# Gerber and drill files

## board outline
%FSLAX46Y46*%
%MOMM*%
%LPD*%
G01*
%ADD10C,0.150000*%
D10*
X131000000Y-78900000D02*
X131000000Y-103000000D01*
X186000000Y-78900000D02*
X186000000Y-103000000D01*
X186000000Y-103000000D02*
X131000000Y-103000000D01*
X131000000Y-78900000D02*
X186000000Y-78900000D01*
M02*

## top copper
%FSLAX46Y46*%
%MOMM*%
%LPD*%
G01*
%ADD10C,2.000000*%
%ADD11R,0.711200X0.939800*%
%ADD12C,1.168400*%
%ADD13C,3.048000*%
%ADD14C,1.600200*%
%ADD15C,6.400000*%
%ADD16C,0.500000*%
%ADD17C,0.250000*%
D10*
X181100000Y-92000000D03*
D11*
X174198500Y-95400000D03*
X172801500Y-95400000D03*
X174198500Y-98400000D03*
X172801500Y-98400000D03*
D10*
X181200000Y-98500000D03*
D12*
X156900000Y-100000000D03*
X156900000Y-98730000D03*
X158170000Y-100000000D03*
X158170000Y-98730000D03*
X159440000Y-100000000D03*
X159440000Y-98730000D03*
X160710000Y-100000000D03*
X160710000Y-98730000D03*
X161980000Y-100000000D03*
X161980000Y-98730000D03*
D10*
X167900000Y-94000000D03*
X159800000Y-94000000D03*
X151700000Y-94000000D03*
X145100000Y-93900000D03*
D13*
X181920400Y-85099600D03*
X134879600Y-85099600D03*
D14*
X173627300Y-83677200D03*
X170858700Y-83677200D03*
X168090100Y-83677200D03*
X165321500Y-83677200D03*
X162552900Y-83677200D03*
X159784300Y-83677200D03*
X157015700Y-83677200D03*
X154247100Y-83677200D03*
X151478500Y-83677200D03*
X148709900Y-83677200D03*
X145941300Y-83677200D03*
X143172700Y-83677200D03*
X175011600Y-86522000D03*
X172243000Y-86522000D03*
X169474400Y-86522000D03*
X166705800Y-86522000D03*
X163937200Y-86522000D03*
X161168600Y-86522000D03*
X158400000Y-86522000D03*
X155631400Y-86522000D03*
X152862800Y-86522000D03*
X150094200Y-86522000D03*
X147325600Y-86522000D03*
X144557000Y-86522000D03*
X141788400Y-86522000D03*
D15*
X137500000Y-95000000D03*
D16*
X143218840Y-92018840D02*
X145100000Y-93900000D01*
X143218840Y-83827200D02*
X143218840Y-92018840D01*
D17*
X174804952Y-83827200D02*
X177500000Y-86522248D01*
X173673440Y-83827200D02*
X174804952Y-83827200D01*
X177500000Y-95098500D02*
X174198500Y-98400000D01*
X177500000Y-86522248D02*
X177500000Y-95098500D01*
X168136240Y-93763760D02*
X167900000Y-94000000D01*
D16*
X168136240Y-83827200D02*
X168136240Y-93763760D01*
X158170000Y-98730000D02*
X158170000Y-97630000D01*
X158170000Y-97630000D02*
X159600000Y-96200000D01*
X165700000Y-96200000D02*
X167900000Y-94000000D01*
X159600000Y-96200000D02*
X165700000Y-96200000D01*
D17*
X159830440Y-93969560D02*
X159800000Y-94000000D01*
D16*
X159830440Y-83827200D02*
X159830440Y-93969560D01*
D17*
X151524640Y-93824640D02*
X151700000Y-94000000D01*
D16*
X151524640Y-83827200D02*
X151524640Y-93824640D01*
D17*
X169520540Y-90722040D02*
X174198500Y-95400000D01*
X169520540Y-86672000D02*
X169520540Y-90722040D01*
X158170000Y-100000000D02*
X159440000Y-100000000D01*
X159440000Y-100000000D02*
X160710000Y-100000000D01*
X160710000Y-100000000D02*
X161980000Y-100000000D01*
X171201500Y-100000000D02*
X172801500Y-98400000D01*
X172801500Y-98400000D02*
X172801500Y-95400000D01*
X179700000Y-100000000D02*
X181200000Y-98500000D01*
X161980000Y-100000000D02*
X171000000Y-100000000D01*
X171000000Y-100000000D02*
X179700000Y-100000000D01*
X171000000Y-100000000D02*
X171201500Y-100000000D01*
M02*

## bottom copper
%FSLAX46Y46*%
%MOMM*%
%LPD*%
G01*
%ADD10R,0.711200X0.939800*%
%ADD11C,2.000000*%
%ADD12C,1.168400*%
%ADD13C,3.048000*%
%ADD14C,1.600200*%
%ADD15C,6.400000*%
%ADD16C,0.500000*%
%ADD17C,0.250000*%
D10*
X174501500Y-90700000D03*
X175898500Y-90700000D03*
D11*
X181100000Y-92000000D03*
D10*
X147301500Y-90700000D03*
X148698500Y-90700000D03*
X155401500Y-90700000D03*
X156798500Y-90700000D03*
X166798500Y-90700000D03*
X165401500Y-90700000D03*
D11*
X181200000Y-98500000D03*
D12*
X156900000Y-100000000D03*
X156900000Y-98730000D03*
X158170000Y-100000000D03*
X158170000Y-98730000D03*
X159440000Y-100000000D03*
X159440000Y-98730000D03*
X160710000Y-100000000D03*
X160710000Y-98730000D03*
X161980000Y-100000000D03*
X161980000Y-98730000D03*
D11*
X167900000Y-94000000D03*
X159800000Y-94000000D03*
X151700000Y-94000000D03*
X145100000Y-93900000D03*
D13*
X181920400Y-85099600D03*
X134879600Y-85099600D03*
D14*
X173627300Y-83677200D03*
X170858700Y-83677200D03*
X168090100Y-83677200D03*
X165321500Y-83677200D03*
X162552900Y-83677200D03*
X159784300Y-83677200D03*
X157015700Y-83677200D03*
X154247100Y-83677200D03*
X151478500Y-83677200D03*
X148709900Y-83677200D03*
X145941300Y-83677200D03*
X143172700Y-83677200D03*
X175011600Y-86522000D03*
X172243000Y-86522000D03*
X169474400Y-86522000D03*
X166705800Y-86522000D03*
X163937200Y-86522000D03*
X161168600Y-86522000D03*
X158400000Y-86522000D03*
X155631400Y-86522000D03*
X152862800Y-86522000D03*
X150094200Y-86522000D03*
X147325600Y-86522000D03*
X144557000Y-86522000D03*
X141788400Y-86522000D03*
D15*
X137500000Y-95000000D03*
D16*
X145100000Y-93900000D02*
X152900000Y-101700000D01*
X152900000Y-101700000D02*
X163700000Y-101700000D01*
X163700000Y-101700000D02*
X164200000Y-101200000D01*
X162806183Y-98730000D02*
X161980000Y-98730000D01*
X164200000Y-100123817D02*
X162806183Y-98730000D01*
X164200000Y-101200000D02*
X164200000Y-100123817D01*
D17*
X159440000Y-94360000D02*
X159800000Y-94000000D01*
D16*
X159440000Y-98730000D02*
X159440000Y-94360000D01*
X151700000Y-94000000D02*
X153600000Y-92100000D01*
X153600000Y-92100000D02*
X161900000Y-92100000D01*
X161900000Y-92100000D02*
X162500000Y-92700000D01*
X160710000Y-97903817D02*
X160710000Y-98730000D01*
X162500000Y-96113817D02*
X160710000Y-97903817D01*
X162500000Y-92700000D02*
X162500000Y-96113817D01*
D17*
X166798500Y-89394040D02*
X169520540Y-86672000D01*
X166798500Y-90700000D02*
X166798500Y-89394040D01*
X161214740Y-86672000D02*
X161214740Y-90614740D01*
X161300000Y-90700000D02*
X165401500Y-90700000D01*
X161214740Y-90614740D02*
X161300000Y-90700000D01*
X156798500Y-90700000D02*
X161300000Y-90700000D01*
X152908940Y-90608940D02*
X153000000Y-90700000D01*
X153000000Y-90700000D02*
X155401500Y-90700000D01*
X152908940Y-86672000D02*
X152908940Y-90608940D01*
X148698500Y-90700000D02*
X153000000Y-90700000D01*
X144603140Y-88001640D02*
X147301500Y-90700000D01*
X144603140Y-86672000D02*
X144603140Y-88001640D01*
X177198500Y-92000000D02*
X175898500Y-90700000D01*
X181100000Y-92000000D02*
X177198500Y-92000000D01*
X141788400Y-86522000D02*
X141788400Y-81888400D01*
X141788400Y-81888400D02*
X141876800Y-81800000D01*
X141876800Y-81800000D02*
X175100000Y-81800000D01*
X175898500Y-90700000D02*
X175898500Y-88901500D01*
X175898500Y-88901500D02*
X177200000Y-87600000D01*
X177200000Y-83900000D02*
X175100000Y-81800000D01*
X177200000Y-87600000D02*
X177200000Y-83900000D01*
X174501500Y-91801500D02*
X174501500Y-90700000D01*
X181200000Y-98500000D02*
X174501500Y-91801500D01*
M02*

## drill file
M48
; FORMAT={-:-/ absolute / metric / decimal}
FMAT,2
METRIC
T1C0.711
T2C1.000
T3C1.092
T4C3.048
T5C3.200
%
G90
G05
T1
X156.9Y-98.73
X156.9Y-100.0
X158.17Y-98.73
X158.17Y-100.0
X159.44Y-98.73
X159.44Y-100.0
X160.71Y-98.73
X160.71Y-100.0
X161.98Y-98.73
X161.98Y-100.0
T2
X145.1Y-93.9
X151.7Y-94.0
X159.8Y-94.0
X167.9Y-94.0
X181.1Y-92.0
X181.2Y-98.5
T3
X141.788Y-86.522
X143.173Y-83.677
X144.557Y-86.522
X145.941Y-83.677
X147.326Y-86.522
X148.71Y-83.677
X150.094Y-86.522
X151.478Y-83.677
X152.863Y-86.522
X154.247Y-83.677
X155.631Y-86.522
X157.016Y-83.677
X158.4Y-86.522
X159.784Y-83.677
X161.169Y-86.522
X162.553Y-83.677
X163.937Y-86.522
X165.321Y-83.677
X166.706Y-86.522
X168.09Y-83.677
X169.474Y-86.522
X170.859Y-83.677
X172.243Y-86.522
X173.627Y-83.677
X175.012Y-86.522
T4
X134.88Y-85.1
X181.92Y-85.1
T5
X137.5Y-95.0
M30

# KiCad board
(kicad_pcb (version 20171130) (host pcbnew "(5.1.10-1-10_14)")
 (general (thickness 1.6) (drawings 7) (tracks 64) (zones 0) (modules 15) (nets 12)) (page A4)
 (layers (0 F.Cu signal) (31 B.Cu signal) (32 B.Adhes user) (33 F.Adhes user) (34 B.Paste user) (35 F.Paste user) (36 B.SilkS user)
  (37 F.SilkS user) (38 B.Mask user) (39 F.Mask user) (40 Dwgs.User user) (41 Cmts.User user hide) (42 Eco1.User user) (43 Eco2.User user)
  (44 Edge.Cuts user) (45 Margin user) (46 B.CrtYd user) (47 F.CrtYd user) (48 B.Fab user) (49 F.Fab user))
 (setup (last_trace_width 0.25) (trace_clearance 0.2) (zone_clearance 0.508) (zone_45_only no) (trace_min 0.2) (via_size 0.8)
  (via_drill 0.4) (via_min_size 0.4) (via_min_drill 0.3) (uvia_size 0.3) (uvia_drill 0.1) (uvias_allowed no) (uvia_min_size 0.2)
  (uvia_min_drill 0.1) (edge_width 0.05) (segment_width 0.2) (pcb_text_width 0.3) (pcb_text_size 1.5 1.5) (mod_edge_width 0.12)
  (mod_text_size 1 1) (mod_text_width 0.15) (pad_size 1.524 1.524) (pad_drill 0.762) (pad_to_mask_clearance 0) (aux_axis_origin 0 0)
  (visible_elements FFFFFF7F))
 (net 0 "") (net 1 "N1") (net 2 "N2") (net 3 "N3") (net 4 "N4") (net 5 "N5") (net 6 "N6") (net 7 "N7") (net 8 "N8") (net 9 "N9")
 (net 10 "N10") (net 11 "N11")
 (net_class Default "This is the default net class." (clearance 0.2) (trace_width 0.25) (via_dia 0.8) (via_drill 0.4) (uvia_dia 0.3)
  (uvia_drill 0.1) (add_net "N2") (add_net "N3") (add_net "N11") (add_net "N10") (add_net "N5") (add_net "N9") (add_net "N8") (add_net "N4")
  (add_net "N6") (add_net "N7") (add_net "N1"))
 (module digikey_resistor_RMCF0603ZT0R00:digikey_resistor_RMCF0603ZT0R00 (layer B.Cu) (at 175.2 90.7 180)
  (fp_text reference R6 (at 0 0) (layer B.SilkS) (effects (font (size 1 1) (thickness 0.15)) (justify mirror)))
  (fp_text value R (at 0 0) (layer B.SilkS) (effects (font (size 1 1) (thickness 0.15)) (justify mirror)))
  (pad 2 smd rect (at 0.6985 0 180) (size 0.7112 0.9398) (layers B.Cu B.Paste B.Mask) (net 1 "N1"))
  (pad 1 smd rect (at -0.6985 0 180) (size 0.7112 0.9398) (layers B.Cu B.Paste B.Mask) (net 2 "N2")))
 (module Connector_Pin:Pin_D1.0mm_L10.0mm (layer F.Cu) (at 181.1 92)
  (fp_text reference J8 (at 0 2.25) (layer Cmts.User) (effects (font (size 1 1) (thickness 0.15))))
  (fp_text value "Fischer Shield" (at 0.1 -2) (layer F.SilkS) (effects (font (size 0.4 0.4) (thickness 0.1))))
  (pad 1 thru_hole circle (at 0 0) (size 2 2) (drill 1) (layers *.Cu *.Mask) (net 2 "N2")))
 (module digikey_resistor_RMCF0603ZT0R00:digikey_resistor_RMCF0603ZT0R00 (layer F.Cu) (at 173.5 95.4)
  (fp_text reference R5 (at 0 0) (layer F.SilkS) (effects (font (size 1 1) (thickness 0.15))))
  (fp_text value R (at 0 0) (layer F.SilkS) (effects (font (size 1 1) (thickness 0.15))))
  (pad 2 smd rect (at 0.6985 0) (size 0.7112 0.9398) (layers F.Cu F.Paste F.Mask) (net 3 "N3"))
  (pad 1 smd rect (at -0.6985 0) (size 0.7112 0.9398) (layers F.Cu F.Paste F.Mask) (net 1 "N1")))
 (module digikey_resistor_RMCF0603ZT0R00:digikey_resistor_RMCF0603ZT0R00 (layer F.Cu) (at 173.5 98.4)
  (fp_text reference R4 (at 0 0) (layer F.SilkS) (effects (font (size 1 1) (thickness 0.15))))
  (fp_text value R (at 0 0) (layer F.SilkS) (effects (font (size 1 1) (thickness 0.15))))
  (pad 2 smd rect (at 0.6985 0) (size 0.7112 0.9398) (layers F.Cu F.Paste F.Mask) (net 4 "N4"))
  (pad 1 smd rect (at -0.6985 0) (size 0.7112 0.9398) (layers F.Cu F.Paste F.Mask) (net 1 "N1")))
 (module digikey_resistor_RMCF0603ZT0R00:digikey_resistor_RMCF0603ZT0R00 (layer B.Cu) (at 148 90.7 180)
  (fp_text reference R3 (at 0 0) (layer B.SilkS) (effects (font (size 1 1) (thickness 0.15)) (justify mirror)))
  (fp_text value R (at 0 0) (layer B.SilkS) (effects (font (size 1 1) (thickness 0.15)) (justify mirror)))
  (pad 2 smd rect (at 0.6985 0 180) (size 0.7112 0.9398) (layers B.Cu B.Paste B.Mask) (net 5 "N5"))
  (pad 1 smd rect (at -0.6985 0 180) (size 0.7112 0.9398) (layers B.Cu B.Paste B.Mask) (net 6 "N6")))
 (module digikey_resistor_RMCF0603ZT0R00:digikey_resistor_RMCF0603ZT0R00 (layer B.Cu) (at 156.1 90.7 180)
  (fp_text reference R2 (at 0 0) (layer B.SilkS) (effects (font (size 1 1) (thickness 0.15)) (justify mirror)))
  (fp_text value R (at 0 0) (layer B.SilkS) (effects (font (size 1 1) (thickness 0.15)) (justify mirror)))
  (pad 2 smd rect (at 0.6985 0 180) (size 0.7112 0.9398) (layers B.Cu B.Paste B.Mask) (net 6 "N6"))
  (pad 1 smd rect (at -0.6985 0 180) (size 0.7112 0.9398) (layers B.Cu B.Paste B.Mask) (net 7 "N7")))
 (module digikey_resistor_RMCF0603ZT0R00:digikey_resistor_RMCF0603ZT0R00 (layer B.Cu) (at 166.1 90.7)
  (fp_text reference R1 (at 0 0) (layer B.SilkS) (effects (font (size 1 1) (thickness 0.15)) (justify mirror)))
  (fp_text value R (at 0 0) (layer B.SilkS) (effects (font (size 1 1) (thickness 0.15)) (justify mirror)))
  (pad 2 smd rect (at 0.6985 0) (size 0.7112 0.9398) (layers B.Cu B.Paste B.Mask) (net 3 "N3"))
  (pad 1 smd rect (at -0.6985 0) (size 0.7112 0.9398) (layers B.Cu B.Paste B.Mask) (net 7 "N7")))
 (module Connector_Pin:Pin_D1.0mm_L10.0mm (layer F.Cu) (at 181.2 98.5)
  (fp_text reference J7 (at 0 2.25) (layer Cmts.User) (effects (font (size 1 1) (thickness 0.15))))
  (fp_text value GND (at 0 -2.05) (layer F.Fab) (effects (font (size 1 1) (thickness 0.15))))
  (pad 1 thru_hole circle (at 0 0) (size 2 2) (drill 1) (layers *.Cu *.Mask) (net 1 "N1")))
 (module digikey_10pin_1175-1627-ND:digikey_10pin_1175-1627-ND (layer F.Cu) (at 156.9 100)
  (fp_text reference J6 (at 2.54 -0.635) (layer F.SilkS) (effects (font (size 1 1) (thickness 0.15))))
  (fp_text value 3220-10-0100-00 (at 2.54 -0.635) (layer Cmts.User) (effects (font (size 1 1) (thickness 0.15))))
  (pad 1 thru_hole circle (at 0 0) (size 1.1684 1.1684) (drill 0.7112) (layers *.Cu *.Mask))
  (pad 2 thru_hole circle (at 0 -1.27) (size 1.1684 1.1684) (drill 0.7112) (layers *.Cu *.Mask))
  (pad 3 thru_hole circle (at 1.27 0) (size 1.1684 1.1684) (drill 0.7112) (layers *.Cu *.Mask) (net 1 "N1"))
  (pad 4 thru_hole circle (at 1.27 -1.27) (size 1.1684 1.1684) (drill 0.7112) (layers *.Cu *.Mask) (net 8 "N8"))
  (pad 5 thru_hole circle (at 2.54 0) (size 1.1684 1.1684) (drill 0.7112) (layers *.Cu *.Mask) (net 1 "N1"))
  (pad 6 thru_hole circle (at 2.54 -1.27) (size 1.1684 1.1684) (drill 0.7112) (layers *.Cu *.Mask) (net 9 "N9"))
  (pad 7 thru_hole circle (at 3.81 0) (size 1.1684 1.1684) (drill 0.7112) (layers *.Cu *.Mask) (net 1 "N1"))
  (pad 8 thru_hole circle (at 3.81 -1.27) (size 1.1684 1.1684) (drill 0.7112) (layers *.Cu *.Mask) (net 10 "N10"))
  (pad 9 thru_hole circle (at 5.08 0) (size 1.1684 1.1684) (drill 0.7112) (layers *.Cu *.Mask) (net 1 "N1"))
  (pad 10 thru_hole circle (at 5.08 -1.27) (size 1.1684 1.1684) (drill 0.7112) (layers *.Cu *.Mask) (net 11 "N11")))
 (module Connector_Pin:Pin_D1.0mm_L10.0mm (layer F.Cu) (at 167.9 94)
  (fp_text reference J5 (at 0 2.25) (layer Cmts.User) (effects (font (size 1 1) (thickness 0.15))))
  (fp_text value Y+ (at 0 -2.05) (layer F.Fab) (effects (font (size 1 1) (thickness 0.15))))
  (pad 1 thru_hole circle (at 0 0) (size 2 2) (drill 1) (layers *.Cu *.Mask) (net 8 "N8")))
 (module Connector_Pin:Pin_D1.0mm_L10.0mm (layer F.Cu) (at 159.8 94)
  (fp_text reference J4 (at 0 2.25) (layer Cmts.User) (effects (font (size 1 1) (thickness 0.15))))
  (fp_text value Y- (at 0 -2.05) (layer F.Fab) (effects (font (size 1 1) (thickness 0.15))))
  (pad 1 thru_hole circle (at 0 0) (size 2 2) (drill 1) (layers *.Cu *.Mask) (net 9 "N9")))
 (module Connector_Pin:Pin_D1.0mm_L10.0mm (layer F.Cu) (at 151.7 94)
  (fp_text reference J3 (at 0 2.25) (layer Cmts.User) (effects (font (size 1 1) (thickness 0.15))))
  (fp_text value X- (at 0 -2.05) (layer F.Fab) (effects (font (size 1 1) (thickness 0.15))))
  (pad 1 thru_hole circle (at 0 0) (size 2 2) (drill 1) (layers *.Cu *.Mask) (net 10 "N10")))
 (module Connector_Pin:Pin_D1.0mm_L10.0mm (layer F.Cu) (at 145.1 93.9)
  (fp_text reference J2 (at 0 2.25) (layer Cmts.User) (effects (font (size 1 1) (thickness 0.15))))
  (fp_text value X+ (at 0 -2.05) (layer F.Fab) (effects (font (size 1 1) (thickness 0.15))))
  (pad 1 thru_hole circle (at 0 0) (size 2 2) (drill 1) (layers *.Cu *.Mask) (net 11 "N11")))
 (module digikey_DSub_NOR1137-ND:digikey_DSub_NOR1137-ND (layer F.Cu) (at 158.4 75.6)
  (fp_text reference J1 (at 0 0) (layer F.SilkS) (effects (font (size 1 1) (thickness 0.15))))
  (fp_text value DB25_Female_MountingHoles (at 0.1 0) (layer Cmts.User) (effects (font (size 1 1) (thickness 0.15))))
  (pad 27 thru_hole circle (at 23.5204 9.4996) (size 3.048 3.048) (drill 3.048) (layers *.Cu *.Mask))
  (pad 26 thru_hole circle (at -23.5204 9.4996) (size 3.048 3.048) (drill 3.048) (layers *.Cu *.Mask))
  (pad 25 thru_hole circle (at 15.2273 8.0772) (size 1.6002 1.6002) (drill 1.0922) (layers *.Cu *.Mask) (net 4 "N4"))
  (pad 24 thru_hole circle (at 12.4587 8.0772) (size 1.6002 1.6002) (drill 1.0922) (layers *.Cu *.Mask))
  (pad 23 thru_hole circle (at 9.6901 8.0772) (size 1.6002 1.6002) (drill 1.0922) (layers *.Cu *.Mask) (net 8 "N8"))
  (pad 22 thru_hole circle (at 6.9215 8.0772) (size 1.6002 1.6002) (drill 1.0922) (layers *.Cu *.Mask))
  (pad 21 thru_hole circle (at 4.1529 8.0772) (size 1.6002 1.6002) (drill 1.0922) (layers *.Cu *.Mask))
  (pad 20 thru_hole circle (at 1.3843 8.0772) (size 1.6002 1.6002) (drill 1.0922) (layers *.Cu *.Mask) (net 9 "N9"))
  (pad 19 thru_hole circle (at -1.3843 8.0772) (size 1.6002 1.6002) (drill 1.0922) (layers *.Cu *.Mask))
  (pad 18 thru_hole circle (at -4.1529 8.0772) (size 1.6002 1.6002) (drill 1.0922) (layers *.Cu *.Mask))
  (pad 17 thru_hole circle (at -6.9215 8.0772) (size 1.6002 1.6002) (drill 1.0922) (layers *.Cu *.Mask) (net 10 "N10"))
  (pad 16 thru_hole circle (at -9.6901 8.0772) (size 1.6002 1.6002) (drill 1.0922) (layers *.Cu *.Mask))
  (pad 15 thru_hole circle (at -12.4587 8.0772) (size 1.6002 1.6002) (drill 1.0922) (layers *.Cu *.Mask))
  (pad 14 thru_hole circle (at -15.2273 8.0772) (size 1.6002 1.6002) (drill 1.0922) (layers *.Cu *.Mask) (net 11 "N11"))
  (pad 13 thru_hole circle (at 16.6116 10.922) (size 1.6002 1.6002) (drill 1.0922) (layers *.Cu *.Mask))
  (pad 12 thru_hole circle (at 13.843 10.922) (size 1.6002 1.6002) (drill 1.0922) (layers *.Cu *.Mask))
  (pad 11 thru_hole circle (at 11.0744 10.922) (size 1.6002 1.6002) (drill 1.0922) (layers *.Cu *.Mask) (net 3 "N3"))
  (pad 10 thru_hole circle (at 8.3058 10.922) (size 1.6002 1.6002) (drill 1.0922) (layers *.Cu *.Mask))
  (pad 9 thru_hole circle (at 5.5372 10.922) (size 1.6002 1.6002) (drill 1.0922) (layers *.Cu *.Mask))
  (pad 8 thru_hole circle (at 2.7686 10.922) (size 1.6002 1.6002) (drill 1.0922) (layers *.Cu *.Mask) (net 7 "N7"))
  (pad 7 thru_hole circle (at 0 10.922) (size 1.6002 1.6002) (drill 1.0922) (layers *.Cu *.Mask))
  (pad 6 thru_hole circle (at -2.7686 10.922) (size 1.6002 1.6002) (drill 1.0922) (layers *.Cu *.Mask))
  (pad 5 thru_hole circle (at -5.5372 10.922) (size 1.6002 1.6002) (drill 1.0922) (layers *.Cu *.Mask) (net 6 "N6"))
  (pad 4 thru_hole circle (at -8.3058 10.922) (size 1.6002 1.6002) (drill 1.0922) (layers *.Cu *.Mask))
  (pad 3 thru_hole circle (at -11.0744 10.922) (size 1.6002 1.6002) (drill 1.0922) (layers *.Cu *.Mask))
  (pad 2 thru_hole circle (at -13.843 10.922) (size 1.6002 1.6002) (drill 1.0922) (layers *.Cu *.Mask) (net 5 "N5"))
  (pad 1 thru_hole circle (at -16.6116 10.922) (size 1.6002 1.6002) (drill 1.0922) (layers *.Cu *.Mask) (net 2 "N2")))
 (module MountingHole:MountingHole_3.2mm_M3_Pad (layer F.Cu) (at 137.5 95)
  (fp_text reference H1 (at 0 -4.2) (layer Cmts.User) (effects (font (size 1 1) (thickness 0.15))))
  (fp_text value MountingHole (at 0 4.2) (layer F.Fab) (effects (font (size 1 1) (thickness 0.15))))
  (pad 1 thru_hole circle (at 0 0) (size 6.4 6.4) (drill 3.2) (layers *.Cu *.Mask)))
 (gr_line (start 131 78.9) (end 131 103) (layer Edge.Cuts) (width 0.15))
 (gr_line (start 186 78.9) (end 186 103) (layer Edge.Cuts) (width 0.15))
 (gr_line (start 186 103) (end 131 103) (layer Edge.Cuts) (width 0.15))
 (gr_line (start 131 78.9) (end 186 78.9) (layer Edge.Cuts) (width 0.15))
 (segment (start 143.21884 92.01884) (end 145.1 93.9) (width 0.5) (layer F.Cu) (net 11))
 (segment (start 143.21884 83.8272) (end 143.21884 92.01884) (width 0.5) (layer F.Cu) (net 11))
 (segment (start 145.1 93.9) (end 152.9 101.7) (width 0.5) (layer B.Cu) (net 11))
 (segment (start 152.9 101.7) (end 163.7 101.7) (width 0.5) (layer B.Cu) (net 11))
 (segment (start 163.7 101.7) (end 164.2 101.2) (width 0.5) (layer B.Cu) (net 11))
 (segment (start 162.806183 98.73) (end 161.98 98.73) (width 0.5) (layer B.Cu) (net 11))
 (segment (start 164.2 100.123817) (end 162.806183 98.73) (width 0.5) (layer B.Cu) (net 11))
 (segment (start 164.2 101.2) (end 164.2 100.123817) (width 0.5) (layer B.Cu) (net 11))
 (segment (start 174.804952 83.8272) (end 177.5 86.522248) (width 0.25) (layer F.Cu) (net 4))
 (segment (start 173.67344 83.8272) (end 174.804952 83.8272) (width 0.25) (layer F.Cu) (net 4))
 (segment (start 177.5 95.0985) (end 174.1985 98.4) (width 0.25) (layer F.Cu) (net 4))
 (segment (start 177.5 86.522248) (end 177.5 95.0985) (width 0.25) (layer F.Cu) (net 4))
 (segment (start 168.13624 93.76376) (end 167.9 94) (width 0.25) (layer F.Cu) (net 8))
 (segment (start 168.13624 83.8272) (end 168.13624 93.76376) (width 0.5) (layer F.Cu) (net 8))
 (segment (start 158.17 98.73) (end 158.17 97.63) (width 0.5) (layer F.Cu) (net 8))
 (segment (start 158.17 97.63) (end 159.6 96.2) (width 0.5) (layer F.Cu) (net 8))
 (segment (start 165.7 96.2) (end 167.9 94) (width 0.5) (layer F.Cu) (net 8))
 (segment (start 159.6 96.2) (end 165.7 96.2) (width 0.5) (layer F.Cu) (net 8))
 (segment (start 159.83044 93.96956) (end 159.8 94) (width 0.25) (layer F.Cu) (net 9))
 (segment (start 159.83044 83.8272) (end 159.83044 93.96956) (width 0.5) (layer F.Cu) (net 9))
 (segment (start 159.44 94.36) (end 159.8 94) (width 0.25) (layer B.Cu) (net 9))
 (segment (start 159.44 98.73) (end 159.44 94.36) (width 0.5) (layer B.Cu) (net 9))
 (segment (start 151.52464 93.82464) (end 151.7 94) (width 0.25) (layer F.Cu) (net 10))
 (segment (start 151.52464 83.8272) (end 151.52464 93.82464) (width 0.5) (layer F.Cu) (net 10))
 (segment (start 151.7 94) (end 153.6 92.1) (width 0.5) (layer B.Cu) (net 10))
 (segment (start 153.6 92.1) (end 161.9 92.1) (width 0.5) (layer B.Cu) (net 10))
 (segment (start 161.9 92.1) (end 162.5 92.7) (width 0.5) (layer B.Cu) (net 10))
 (segment (start 160.71 97.903817) (end 160.71 98.73) (width 0.5) (layer B.Cu) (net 10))
 (segment (start 162.5 96.113817) (end 160.71 97.903817) (width 0.5) (layer B.Cu) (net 10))
 (segment (start 162.5 92.7) (end 162.5 96.113817) (width 0.5) (layer B.Cu) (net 10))
 (segment (start 166.7985 89.39404) (end 169.52054 86.672) (width 0.25) (layer B.Cu) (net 3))
 (segment (start 166.7985 90.7) (end 166.7985 89.39404) (width 0.25) (layer B.Cu) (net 3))
 (segment (start 169.52054 90.72204) (end 174.1985 95.4) (width 0.25) (layer F.Cu) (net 3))
 (segment (start 169.52054 86.672) (end 169.52054 90.72204) (width 0.25) (layer F.Cu) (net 3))
 (segment (start 161.21474 86.672) (end 161.21474 90.61474) (width 0.25) (layer B.Cu) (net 7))
 (segment (start 161.3 90.7) (end 165.4015 90.7) (width 0.25) (layer B.Cu) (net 7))
 (segment (start 161.21474 90.61474) (end 161.3 90.7) (width 0.25) (layer B.Cu) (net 7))
 (segment (start 156.7985 90.7) (end 161.3 90.7) (width 0.25) (layer B.Cu) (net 7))
 (segment (start 152.90894 90.60894) (end 153 90.7) (width 0.25) (layer B.Cu) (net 6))
 (segment (start 153 90.7) (end 155.4015 90.7) (width 0.25) (layer B.Cu) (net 6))
 (segment (start 152.90894 86.672) (end 152.90894 90.60894) (width 0.25) (layer B.Cu) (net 6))
 (segment (start 148.6985 90.7) (end 153 90.7) (width 0.25) (layer B.Cu) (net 6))
 (segment (start 144.60314 88.00164) (end 147.3015 90.7) (width 0.25) (layer B.Cu) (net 5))
 (segment (start 144.60314 86.672) (end 144.60314 88.00164) (width 0.25) (layer B.Cu) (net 5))
 (segment (start 177.1985 92) (end 175.8985 90.7) (width 0.25) (layer B.Cu) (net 2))
 (segment (start 181.1 92) (end 177.1985 92) (width 0.25) (layer B.Cu) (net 2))
 (segment (start 141.7884 86.522) (end 141.7884 81.8884) (width 0.25) (layer B.Cu) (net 2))
 (segment (start 141.7884 81.8884) (end 141.8768 81.8) (width 0.25) (layer B.Cu) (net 2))
 (segment (start 141.8768 81.8) (end 175.1 81.8) (width 0.25) (layer B.Cu) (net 2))
 (segment (start 175.8985 90.7) (end 175.8985 88.9015) (width 0.25) (layer B.Cu) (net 2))
 (segment (start 175.8985 88.9015) (end 177.2 87.6) (width 0.25) (layer B.Cu) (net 2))
 (segment (start 177.2 83.9) (end 175.1 81.8) (width 0.25) (layer B.Cu) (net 2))
 (segment (start 177.2 87.6) (end 177.2 83.9) (width 0.25) (layer B.Cu) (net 2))
 (segment (start 158.17 100) (end 159.44 100) (width 0.25) (layer F.Cu) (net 1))
 (segment (start 159.44 100) (end 160.71 100) (width 0.25) (layer F.Cu) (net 1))
 (segment (start 160.71 100) (end 161.98 100) (width 0.25) (layer F.Cu) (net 1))
 (segment (start 171.2015 100) (end 172.8015 98.4) (width 0.25) (layer F.Cu) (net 1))
 (segment (start 172.8015 98.4) (end 172.8015 95.4) (width 0.25) (layer F.Cu) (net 1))
 (segment (start 179.7 100) (end 181.2 98.5) (width 0.25) (layer F.Cu) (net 1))
 (segment (start 161.98 100) (end 171 100) (width 0.25) (layer F.Cu) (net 1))
 (segment (start 171 100) (end 179.7 100) (width 0.25) (layer F.Cu) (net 1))
 (segment (start 171 100) (end 171.2015 100) (width 0.25) (layer F.Cu) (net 1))
 (segment (start 174.5015 91.8015) (end 174.5015 90.7) (width 0.25) (layer B.Cu) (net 1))
 (segment (start 181.2 98.5) (end 174.5015 91.8015) (width 0.25) (layer B.Cu) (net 1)))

